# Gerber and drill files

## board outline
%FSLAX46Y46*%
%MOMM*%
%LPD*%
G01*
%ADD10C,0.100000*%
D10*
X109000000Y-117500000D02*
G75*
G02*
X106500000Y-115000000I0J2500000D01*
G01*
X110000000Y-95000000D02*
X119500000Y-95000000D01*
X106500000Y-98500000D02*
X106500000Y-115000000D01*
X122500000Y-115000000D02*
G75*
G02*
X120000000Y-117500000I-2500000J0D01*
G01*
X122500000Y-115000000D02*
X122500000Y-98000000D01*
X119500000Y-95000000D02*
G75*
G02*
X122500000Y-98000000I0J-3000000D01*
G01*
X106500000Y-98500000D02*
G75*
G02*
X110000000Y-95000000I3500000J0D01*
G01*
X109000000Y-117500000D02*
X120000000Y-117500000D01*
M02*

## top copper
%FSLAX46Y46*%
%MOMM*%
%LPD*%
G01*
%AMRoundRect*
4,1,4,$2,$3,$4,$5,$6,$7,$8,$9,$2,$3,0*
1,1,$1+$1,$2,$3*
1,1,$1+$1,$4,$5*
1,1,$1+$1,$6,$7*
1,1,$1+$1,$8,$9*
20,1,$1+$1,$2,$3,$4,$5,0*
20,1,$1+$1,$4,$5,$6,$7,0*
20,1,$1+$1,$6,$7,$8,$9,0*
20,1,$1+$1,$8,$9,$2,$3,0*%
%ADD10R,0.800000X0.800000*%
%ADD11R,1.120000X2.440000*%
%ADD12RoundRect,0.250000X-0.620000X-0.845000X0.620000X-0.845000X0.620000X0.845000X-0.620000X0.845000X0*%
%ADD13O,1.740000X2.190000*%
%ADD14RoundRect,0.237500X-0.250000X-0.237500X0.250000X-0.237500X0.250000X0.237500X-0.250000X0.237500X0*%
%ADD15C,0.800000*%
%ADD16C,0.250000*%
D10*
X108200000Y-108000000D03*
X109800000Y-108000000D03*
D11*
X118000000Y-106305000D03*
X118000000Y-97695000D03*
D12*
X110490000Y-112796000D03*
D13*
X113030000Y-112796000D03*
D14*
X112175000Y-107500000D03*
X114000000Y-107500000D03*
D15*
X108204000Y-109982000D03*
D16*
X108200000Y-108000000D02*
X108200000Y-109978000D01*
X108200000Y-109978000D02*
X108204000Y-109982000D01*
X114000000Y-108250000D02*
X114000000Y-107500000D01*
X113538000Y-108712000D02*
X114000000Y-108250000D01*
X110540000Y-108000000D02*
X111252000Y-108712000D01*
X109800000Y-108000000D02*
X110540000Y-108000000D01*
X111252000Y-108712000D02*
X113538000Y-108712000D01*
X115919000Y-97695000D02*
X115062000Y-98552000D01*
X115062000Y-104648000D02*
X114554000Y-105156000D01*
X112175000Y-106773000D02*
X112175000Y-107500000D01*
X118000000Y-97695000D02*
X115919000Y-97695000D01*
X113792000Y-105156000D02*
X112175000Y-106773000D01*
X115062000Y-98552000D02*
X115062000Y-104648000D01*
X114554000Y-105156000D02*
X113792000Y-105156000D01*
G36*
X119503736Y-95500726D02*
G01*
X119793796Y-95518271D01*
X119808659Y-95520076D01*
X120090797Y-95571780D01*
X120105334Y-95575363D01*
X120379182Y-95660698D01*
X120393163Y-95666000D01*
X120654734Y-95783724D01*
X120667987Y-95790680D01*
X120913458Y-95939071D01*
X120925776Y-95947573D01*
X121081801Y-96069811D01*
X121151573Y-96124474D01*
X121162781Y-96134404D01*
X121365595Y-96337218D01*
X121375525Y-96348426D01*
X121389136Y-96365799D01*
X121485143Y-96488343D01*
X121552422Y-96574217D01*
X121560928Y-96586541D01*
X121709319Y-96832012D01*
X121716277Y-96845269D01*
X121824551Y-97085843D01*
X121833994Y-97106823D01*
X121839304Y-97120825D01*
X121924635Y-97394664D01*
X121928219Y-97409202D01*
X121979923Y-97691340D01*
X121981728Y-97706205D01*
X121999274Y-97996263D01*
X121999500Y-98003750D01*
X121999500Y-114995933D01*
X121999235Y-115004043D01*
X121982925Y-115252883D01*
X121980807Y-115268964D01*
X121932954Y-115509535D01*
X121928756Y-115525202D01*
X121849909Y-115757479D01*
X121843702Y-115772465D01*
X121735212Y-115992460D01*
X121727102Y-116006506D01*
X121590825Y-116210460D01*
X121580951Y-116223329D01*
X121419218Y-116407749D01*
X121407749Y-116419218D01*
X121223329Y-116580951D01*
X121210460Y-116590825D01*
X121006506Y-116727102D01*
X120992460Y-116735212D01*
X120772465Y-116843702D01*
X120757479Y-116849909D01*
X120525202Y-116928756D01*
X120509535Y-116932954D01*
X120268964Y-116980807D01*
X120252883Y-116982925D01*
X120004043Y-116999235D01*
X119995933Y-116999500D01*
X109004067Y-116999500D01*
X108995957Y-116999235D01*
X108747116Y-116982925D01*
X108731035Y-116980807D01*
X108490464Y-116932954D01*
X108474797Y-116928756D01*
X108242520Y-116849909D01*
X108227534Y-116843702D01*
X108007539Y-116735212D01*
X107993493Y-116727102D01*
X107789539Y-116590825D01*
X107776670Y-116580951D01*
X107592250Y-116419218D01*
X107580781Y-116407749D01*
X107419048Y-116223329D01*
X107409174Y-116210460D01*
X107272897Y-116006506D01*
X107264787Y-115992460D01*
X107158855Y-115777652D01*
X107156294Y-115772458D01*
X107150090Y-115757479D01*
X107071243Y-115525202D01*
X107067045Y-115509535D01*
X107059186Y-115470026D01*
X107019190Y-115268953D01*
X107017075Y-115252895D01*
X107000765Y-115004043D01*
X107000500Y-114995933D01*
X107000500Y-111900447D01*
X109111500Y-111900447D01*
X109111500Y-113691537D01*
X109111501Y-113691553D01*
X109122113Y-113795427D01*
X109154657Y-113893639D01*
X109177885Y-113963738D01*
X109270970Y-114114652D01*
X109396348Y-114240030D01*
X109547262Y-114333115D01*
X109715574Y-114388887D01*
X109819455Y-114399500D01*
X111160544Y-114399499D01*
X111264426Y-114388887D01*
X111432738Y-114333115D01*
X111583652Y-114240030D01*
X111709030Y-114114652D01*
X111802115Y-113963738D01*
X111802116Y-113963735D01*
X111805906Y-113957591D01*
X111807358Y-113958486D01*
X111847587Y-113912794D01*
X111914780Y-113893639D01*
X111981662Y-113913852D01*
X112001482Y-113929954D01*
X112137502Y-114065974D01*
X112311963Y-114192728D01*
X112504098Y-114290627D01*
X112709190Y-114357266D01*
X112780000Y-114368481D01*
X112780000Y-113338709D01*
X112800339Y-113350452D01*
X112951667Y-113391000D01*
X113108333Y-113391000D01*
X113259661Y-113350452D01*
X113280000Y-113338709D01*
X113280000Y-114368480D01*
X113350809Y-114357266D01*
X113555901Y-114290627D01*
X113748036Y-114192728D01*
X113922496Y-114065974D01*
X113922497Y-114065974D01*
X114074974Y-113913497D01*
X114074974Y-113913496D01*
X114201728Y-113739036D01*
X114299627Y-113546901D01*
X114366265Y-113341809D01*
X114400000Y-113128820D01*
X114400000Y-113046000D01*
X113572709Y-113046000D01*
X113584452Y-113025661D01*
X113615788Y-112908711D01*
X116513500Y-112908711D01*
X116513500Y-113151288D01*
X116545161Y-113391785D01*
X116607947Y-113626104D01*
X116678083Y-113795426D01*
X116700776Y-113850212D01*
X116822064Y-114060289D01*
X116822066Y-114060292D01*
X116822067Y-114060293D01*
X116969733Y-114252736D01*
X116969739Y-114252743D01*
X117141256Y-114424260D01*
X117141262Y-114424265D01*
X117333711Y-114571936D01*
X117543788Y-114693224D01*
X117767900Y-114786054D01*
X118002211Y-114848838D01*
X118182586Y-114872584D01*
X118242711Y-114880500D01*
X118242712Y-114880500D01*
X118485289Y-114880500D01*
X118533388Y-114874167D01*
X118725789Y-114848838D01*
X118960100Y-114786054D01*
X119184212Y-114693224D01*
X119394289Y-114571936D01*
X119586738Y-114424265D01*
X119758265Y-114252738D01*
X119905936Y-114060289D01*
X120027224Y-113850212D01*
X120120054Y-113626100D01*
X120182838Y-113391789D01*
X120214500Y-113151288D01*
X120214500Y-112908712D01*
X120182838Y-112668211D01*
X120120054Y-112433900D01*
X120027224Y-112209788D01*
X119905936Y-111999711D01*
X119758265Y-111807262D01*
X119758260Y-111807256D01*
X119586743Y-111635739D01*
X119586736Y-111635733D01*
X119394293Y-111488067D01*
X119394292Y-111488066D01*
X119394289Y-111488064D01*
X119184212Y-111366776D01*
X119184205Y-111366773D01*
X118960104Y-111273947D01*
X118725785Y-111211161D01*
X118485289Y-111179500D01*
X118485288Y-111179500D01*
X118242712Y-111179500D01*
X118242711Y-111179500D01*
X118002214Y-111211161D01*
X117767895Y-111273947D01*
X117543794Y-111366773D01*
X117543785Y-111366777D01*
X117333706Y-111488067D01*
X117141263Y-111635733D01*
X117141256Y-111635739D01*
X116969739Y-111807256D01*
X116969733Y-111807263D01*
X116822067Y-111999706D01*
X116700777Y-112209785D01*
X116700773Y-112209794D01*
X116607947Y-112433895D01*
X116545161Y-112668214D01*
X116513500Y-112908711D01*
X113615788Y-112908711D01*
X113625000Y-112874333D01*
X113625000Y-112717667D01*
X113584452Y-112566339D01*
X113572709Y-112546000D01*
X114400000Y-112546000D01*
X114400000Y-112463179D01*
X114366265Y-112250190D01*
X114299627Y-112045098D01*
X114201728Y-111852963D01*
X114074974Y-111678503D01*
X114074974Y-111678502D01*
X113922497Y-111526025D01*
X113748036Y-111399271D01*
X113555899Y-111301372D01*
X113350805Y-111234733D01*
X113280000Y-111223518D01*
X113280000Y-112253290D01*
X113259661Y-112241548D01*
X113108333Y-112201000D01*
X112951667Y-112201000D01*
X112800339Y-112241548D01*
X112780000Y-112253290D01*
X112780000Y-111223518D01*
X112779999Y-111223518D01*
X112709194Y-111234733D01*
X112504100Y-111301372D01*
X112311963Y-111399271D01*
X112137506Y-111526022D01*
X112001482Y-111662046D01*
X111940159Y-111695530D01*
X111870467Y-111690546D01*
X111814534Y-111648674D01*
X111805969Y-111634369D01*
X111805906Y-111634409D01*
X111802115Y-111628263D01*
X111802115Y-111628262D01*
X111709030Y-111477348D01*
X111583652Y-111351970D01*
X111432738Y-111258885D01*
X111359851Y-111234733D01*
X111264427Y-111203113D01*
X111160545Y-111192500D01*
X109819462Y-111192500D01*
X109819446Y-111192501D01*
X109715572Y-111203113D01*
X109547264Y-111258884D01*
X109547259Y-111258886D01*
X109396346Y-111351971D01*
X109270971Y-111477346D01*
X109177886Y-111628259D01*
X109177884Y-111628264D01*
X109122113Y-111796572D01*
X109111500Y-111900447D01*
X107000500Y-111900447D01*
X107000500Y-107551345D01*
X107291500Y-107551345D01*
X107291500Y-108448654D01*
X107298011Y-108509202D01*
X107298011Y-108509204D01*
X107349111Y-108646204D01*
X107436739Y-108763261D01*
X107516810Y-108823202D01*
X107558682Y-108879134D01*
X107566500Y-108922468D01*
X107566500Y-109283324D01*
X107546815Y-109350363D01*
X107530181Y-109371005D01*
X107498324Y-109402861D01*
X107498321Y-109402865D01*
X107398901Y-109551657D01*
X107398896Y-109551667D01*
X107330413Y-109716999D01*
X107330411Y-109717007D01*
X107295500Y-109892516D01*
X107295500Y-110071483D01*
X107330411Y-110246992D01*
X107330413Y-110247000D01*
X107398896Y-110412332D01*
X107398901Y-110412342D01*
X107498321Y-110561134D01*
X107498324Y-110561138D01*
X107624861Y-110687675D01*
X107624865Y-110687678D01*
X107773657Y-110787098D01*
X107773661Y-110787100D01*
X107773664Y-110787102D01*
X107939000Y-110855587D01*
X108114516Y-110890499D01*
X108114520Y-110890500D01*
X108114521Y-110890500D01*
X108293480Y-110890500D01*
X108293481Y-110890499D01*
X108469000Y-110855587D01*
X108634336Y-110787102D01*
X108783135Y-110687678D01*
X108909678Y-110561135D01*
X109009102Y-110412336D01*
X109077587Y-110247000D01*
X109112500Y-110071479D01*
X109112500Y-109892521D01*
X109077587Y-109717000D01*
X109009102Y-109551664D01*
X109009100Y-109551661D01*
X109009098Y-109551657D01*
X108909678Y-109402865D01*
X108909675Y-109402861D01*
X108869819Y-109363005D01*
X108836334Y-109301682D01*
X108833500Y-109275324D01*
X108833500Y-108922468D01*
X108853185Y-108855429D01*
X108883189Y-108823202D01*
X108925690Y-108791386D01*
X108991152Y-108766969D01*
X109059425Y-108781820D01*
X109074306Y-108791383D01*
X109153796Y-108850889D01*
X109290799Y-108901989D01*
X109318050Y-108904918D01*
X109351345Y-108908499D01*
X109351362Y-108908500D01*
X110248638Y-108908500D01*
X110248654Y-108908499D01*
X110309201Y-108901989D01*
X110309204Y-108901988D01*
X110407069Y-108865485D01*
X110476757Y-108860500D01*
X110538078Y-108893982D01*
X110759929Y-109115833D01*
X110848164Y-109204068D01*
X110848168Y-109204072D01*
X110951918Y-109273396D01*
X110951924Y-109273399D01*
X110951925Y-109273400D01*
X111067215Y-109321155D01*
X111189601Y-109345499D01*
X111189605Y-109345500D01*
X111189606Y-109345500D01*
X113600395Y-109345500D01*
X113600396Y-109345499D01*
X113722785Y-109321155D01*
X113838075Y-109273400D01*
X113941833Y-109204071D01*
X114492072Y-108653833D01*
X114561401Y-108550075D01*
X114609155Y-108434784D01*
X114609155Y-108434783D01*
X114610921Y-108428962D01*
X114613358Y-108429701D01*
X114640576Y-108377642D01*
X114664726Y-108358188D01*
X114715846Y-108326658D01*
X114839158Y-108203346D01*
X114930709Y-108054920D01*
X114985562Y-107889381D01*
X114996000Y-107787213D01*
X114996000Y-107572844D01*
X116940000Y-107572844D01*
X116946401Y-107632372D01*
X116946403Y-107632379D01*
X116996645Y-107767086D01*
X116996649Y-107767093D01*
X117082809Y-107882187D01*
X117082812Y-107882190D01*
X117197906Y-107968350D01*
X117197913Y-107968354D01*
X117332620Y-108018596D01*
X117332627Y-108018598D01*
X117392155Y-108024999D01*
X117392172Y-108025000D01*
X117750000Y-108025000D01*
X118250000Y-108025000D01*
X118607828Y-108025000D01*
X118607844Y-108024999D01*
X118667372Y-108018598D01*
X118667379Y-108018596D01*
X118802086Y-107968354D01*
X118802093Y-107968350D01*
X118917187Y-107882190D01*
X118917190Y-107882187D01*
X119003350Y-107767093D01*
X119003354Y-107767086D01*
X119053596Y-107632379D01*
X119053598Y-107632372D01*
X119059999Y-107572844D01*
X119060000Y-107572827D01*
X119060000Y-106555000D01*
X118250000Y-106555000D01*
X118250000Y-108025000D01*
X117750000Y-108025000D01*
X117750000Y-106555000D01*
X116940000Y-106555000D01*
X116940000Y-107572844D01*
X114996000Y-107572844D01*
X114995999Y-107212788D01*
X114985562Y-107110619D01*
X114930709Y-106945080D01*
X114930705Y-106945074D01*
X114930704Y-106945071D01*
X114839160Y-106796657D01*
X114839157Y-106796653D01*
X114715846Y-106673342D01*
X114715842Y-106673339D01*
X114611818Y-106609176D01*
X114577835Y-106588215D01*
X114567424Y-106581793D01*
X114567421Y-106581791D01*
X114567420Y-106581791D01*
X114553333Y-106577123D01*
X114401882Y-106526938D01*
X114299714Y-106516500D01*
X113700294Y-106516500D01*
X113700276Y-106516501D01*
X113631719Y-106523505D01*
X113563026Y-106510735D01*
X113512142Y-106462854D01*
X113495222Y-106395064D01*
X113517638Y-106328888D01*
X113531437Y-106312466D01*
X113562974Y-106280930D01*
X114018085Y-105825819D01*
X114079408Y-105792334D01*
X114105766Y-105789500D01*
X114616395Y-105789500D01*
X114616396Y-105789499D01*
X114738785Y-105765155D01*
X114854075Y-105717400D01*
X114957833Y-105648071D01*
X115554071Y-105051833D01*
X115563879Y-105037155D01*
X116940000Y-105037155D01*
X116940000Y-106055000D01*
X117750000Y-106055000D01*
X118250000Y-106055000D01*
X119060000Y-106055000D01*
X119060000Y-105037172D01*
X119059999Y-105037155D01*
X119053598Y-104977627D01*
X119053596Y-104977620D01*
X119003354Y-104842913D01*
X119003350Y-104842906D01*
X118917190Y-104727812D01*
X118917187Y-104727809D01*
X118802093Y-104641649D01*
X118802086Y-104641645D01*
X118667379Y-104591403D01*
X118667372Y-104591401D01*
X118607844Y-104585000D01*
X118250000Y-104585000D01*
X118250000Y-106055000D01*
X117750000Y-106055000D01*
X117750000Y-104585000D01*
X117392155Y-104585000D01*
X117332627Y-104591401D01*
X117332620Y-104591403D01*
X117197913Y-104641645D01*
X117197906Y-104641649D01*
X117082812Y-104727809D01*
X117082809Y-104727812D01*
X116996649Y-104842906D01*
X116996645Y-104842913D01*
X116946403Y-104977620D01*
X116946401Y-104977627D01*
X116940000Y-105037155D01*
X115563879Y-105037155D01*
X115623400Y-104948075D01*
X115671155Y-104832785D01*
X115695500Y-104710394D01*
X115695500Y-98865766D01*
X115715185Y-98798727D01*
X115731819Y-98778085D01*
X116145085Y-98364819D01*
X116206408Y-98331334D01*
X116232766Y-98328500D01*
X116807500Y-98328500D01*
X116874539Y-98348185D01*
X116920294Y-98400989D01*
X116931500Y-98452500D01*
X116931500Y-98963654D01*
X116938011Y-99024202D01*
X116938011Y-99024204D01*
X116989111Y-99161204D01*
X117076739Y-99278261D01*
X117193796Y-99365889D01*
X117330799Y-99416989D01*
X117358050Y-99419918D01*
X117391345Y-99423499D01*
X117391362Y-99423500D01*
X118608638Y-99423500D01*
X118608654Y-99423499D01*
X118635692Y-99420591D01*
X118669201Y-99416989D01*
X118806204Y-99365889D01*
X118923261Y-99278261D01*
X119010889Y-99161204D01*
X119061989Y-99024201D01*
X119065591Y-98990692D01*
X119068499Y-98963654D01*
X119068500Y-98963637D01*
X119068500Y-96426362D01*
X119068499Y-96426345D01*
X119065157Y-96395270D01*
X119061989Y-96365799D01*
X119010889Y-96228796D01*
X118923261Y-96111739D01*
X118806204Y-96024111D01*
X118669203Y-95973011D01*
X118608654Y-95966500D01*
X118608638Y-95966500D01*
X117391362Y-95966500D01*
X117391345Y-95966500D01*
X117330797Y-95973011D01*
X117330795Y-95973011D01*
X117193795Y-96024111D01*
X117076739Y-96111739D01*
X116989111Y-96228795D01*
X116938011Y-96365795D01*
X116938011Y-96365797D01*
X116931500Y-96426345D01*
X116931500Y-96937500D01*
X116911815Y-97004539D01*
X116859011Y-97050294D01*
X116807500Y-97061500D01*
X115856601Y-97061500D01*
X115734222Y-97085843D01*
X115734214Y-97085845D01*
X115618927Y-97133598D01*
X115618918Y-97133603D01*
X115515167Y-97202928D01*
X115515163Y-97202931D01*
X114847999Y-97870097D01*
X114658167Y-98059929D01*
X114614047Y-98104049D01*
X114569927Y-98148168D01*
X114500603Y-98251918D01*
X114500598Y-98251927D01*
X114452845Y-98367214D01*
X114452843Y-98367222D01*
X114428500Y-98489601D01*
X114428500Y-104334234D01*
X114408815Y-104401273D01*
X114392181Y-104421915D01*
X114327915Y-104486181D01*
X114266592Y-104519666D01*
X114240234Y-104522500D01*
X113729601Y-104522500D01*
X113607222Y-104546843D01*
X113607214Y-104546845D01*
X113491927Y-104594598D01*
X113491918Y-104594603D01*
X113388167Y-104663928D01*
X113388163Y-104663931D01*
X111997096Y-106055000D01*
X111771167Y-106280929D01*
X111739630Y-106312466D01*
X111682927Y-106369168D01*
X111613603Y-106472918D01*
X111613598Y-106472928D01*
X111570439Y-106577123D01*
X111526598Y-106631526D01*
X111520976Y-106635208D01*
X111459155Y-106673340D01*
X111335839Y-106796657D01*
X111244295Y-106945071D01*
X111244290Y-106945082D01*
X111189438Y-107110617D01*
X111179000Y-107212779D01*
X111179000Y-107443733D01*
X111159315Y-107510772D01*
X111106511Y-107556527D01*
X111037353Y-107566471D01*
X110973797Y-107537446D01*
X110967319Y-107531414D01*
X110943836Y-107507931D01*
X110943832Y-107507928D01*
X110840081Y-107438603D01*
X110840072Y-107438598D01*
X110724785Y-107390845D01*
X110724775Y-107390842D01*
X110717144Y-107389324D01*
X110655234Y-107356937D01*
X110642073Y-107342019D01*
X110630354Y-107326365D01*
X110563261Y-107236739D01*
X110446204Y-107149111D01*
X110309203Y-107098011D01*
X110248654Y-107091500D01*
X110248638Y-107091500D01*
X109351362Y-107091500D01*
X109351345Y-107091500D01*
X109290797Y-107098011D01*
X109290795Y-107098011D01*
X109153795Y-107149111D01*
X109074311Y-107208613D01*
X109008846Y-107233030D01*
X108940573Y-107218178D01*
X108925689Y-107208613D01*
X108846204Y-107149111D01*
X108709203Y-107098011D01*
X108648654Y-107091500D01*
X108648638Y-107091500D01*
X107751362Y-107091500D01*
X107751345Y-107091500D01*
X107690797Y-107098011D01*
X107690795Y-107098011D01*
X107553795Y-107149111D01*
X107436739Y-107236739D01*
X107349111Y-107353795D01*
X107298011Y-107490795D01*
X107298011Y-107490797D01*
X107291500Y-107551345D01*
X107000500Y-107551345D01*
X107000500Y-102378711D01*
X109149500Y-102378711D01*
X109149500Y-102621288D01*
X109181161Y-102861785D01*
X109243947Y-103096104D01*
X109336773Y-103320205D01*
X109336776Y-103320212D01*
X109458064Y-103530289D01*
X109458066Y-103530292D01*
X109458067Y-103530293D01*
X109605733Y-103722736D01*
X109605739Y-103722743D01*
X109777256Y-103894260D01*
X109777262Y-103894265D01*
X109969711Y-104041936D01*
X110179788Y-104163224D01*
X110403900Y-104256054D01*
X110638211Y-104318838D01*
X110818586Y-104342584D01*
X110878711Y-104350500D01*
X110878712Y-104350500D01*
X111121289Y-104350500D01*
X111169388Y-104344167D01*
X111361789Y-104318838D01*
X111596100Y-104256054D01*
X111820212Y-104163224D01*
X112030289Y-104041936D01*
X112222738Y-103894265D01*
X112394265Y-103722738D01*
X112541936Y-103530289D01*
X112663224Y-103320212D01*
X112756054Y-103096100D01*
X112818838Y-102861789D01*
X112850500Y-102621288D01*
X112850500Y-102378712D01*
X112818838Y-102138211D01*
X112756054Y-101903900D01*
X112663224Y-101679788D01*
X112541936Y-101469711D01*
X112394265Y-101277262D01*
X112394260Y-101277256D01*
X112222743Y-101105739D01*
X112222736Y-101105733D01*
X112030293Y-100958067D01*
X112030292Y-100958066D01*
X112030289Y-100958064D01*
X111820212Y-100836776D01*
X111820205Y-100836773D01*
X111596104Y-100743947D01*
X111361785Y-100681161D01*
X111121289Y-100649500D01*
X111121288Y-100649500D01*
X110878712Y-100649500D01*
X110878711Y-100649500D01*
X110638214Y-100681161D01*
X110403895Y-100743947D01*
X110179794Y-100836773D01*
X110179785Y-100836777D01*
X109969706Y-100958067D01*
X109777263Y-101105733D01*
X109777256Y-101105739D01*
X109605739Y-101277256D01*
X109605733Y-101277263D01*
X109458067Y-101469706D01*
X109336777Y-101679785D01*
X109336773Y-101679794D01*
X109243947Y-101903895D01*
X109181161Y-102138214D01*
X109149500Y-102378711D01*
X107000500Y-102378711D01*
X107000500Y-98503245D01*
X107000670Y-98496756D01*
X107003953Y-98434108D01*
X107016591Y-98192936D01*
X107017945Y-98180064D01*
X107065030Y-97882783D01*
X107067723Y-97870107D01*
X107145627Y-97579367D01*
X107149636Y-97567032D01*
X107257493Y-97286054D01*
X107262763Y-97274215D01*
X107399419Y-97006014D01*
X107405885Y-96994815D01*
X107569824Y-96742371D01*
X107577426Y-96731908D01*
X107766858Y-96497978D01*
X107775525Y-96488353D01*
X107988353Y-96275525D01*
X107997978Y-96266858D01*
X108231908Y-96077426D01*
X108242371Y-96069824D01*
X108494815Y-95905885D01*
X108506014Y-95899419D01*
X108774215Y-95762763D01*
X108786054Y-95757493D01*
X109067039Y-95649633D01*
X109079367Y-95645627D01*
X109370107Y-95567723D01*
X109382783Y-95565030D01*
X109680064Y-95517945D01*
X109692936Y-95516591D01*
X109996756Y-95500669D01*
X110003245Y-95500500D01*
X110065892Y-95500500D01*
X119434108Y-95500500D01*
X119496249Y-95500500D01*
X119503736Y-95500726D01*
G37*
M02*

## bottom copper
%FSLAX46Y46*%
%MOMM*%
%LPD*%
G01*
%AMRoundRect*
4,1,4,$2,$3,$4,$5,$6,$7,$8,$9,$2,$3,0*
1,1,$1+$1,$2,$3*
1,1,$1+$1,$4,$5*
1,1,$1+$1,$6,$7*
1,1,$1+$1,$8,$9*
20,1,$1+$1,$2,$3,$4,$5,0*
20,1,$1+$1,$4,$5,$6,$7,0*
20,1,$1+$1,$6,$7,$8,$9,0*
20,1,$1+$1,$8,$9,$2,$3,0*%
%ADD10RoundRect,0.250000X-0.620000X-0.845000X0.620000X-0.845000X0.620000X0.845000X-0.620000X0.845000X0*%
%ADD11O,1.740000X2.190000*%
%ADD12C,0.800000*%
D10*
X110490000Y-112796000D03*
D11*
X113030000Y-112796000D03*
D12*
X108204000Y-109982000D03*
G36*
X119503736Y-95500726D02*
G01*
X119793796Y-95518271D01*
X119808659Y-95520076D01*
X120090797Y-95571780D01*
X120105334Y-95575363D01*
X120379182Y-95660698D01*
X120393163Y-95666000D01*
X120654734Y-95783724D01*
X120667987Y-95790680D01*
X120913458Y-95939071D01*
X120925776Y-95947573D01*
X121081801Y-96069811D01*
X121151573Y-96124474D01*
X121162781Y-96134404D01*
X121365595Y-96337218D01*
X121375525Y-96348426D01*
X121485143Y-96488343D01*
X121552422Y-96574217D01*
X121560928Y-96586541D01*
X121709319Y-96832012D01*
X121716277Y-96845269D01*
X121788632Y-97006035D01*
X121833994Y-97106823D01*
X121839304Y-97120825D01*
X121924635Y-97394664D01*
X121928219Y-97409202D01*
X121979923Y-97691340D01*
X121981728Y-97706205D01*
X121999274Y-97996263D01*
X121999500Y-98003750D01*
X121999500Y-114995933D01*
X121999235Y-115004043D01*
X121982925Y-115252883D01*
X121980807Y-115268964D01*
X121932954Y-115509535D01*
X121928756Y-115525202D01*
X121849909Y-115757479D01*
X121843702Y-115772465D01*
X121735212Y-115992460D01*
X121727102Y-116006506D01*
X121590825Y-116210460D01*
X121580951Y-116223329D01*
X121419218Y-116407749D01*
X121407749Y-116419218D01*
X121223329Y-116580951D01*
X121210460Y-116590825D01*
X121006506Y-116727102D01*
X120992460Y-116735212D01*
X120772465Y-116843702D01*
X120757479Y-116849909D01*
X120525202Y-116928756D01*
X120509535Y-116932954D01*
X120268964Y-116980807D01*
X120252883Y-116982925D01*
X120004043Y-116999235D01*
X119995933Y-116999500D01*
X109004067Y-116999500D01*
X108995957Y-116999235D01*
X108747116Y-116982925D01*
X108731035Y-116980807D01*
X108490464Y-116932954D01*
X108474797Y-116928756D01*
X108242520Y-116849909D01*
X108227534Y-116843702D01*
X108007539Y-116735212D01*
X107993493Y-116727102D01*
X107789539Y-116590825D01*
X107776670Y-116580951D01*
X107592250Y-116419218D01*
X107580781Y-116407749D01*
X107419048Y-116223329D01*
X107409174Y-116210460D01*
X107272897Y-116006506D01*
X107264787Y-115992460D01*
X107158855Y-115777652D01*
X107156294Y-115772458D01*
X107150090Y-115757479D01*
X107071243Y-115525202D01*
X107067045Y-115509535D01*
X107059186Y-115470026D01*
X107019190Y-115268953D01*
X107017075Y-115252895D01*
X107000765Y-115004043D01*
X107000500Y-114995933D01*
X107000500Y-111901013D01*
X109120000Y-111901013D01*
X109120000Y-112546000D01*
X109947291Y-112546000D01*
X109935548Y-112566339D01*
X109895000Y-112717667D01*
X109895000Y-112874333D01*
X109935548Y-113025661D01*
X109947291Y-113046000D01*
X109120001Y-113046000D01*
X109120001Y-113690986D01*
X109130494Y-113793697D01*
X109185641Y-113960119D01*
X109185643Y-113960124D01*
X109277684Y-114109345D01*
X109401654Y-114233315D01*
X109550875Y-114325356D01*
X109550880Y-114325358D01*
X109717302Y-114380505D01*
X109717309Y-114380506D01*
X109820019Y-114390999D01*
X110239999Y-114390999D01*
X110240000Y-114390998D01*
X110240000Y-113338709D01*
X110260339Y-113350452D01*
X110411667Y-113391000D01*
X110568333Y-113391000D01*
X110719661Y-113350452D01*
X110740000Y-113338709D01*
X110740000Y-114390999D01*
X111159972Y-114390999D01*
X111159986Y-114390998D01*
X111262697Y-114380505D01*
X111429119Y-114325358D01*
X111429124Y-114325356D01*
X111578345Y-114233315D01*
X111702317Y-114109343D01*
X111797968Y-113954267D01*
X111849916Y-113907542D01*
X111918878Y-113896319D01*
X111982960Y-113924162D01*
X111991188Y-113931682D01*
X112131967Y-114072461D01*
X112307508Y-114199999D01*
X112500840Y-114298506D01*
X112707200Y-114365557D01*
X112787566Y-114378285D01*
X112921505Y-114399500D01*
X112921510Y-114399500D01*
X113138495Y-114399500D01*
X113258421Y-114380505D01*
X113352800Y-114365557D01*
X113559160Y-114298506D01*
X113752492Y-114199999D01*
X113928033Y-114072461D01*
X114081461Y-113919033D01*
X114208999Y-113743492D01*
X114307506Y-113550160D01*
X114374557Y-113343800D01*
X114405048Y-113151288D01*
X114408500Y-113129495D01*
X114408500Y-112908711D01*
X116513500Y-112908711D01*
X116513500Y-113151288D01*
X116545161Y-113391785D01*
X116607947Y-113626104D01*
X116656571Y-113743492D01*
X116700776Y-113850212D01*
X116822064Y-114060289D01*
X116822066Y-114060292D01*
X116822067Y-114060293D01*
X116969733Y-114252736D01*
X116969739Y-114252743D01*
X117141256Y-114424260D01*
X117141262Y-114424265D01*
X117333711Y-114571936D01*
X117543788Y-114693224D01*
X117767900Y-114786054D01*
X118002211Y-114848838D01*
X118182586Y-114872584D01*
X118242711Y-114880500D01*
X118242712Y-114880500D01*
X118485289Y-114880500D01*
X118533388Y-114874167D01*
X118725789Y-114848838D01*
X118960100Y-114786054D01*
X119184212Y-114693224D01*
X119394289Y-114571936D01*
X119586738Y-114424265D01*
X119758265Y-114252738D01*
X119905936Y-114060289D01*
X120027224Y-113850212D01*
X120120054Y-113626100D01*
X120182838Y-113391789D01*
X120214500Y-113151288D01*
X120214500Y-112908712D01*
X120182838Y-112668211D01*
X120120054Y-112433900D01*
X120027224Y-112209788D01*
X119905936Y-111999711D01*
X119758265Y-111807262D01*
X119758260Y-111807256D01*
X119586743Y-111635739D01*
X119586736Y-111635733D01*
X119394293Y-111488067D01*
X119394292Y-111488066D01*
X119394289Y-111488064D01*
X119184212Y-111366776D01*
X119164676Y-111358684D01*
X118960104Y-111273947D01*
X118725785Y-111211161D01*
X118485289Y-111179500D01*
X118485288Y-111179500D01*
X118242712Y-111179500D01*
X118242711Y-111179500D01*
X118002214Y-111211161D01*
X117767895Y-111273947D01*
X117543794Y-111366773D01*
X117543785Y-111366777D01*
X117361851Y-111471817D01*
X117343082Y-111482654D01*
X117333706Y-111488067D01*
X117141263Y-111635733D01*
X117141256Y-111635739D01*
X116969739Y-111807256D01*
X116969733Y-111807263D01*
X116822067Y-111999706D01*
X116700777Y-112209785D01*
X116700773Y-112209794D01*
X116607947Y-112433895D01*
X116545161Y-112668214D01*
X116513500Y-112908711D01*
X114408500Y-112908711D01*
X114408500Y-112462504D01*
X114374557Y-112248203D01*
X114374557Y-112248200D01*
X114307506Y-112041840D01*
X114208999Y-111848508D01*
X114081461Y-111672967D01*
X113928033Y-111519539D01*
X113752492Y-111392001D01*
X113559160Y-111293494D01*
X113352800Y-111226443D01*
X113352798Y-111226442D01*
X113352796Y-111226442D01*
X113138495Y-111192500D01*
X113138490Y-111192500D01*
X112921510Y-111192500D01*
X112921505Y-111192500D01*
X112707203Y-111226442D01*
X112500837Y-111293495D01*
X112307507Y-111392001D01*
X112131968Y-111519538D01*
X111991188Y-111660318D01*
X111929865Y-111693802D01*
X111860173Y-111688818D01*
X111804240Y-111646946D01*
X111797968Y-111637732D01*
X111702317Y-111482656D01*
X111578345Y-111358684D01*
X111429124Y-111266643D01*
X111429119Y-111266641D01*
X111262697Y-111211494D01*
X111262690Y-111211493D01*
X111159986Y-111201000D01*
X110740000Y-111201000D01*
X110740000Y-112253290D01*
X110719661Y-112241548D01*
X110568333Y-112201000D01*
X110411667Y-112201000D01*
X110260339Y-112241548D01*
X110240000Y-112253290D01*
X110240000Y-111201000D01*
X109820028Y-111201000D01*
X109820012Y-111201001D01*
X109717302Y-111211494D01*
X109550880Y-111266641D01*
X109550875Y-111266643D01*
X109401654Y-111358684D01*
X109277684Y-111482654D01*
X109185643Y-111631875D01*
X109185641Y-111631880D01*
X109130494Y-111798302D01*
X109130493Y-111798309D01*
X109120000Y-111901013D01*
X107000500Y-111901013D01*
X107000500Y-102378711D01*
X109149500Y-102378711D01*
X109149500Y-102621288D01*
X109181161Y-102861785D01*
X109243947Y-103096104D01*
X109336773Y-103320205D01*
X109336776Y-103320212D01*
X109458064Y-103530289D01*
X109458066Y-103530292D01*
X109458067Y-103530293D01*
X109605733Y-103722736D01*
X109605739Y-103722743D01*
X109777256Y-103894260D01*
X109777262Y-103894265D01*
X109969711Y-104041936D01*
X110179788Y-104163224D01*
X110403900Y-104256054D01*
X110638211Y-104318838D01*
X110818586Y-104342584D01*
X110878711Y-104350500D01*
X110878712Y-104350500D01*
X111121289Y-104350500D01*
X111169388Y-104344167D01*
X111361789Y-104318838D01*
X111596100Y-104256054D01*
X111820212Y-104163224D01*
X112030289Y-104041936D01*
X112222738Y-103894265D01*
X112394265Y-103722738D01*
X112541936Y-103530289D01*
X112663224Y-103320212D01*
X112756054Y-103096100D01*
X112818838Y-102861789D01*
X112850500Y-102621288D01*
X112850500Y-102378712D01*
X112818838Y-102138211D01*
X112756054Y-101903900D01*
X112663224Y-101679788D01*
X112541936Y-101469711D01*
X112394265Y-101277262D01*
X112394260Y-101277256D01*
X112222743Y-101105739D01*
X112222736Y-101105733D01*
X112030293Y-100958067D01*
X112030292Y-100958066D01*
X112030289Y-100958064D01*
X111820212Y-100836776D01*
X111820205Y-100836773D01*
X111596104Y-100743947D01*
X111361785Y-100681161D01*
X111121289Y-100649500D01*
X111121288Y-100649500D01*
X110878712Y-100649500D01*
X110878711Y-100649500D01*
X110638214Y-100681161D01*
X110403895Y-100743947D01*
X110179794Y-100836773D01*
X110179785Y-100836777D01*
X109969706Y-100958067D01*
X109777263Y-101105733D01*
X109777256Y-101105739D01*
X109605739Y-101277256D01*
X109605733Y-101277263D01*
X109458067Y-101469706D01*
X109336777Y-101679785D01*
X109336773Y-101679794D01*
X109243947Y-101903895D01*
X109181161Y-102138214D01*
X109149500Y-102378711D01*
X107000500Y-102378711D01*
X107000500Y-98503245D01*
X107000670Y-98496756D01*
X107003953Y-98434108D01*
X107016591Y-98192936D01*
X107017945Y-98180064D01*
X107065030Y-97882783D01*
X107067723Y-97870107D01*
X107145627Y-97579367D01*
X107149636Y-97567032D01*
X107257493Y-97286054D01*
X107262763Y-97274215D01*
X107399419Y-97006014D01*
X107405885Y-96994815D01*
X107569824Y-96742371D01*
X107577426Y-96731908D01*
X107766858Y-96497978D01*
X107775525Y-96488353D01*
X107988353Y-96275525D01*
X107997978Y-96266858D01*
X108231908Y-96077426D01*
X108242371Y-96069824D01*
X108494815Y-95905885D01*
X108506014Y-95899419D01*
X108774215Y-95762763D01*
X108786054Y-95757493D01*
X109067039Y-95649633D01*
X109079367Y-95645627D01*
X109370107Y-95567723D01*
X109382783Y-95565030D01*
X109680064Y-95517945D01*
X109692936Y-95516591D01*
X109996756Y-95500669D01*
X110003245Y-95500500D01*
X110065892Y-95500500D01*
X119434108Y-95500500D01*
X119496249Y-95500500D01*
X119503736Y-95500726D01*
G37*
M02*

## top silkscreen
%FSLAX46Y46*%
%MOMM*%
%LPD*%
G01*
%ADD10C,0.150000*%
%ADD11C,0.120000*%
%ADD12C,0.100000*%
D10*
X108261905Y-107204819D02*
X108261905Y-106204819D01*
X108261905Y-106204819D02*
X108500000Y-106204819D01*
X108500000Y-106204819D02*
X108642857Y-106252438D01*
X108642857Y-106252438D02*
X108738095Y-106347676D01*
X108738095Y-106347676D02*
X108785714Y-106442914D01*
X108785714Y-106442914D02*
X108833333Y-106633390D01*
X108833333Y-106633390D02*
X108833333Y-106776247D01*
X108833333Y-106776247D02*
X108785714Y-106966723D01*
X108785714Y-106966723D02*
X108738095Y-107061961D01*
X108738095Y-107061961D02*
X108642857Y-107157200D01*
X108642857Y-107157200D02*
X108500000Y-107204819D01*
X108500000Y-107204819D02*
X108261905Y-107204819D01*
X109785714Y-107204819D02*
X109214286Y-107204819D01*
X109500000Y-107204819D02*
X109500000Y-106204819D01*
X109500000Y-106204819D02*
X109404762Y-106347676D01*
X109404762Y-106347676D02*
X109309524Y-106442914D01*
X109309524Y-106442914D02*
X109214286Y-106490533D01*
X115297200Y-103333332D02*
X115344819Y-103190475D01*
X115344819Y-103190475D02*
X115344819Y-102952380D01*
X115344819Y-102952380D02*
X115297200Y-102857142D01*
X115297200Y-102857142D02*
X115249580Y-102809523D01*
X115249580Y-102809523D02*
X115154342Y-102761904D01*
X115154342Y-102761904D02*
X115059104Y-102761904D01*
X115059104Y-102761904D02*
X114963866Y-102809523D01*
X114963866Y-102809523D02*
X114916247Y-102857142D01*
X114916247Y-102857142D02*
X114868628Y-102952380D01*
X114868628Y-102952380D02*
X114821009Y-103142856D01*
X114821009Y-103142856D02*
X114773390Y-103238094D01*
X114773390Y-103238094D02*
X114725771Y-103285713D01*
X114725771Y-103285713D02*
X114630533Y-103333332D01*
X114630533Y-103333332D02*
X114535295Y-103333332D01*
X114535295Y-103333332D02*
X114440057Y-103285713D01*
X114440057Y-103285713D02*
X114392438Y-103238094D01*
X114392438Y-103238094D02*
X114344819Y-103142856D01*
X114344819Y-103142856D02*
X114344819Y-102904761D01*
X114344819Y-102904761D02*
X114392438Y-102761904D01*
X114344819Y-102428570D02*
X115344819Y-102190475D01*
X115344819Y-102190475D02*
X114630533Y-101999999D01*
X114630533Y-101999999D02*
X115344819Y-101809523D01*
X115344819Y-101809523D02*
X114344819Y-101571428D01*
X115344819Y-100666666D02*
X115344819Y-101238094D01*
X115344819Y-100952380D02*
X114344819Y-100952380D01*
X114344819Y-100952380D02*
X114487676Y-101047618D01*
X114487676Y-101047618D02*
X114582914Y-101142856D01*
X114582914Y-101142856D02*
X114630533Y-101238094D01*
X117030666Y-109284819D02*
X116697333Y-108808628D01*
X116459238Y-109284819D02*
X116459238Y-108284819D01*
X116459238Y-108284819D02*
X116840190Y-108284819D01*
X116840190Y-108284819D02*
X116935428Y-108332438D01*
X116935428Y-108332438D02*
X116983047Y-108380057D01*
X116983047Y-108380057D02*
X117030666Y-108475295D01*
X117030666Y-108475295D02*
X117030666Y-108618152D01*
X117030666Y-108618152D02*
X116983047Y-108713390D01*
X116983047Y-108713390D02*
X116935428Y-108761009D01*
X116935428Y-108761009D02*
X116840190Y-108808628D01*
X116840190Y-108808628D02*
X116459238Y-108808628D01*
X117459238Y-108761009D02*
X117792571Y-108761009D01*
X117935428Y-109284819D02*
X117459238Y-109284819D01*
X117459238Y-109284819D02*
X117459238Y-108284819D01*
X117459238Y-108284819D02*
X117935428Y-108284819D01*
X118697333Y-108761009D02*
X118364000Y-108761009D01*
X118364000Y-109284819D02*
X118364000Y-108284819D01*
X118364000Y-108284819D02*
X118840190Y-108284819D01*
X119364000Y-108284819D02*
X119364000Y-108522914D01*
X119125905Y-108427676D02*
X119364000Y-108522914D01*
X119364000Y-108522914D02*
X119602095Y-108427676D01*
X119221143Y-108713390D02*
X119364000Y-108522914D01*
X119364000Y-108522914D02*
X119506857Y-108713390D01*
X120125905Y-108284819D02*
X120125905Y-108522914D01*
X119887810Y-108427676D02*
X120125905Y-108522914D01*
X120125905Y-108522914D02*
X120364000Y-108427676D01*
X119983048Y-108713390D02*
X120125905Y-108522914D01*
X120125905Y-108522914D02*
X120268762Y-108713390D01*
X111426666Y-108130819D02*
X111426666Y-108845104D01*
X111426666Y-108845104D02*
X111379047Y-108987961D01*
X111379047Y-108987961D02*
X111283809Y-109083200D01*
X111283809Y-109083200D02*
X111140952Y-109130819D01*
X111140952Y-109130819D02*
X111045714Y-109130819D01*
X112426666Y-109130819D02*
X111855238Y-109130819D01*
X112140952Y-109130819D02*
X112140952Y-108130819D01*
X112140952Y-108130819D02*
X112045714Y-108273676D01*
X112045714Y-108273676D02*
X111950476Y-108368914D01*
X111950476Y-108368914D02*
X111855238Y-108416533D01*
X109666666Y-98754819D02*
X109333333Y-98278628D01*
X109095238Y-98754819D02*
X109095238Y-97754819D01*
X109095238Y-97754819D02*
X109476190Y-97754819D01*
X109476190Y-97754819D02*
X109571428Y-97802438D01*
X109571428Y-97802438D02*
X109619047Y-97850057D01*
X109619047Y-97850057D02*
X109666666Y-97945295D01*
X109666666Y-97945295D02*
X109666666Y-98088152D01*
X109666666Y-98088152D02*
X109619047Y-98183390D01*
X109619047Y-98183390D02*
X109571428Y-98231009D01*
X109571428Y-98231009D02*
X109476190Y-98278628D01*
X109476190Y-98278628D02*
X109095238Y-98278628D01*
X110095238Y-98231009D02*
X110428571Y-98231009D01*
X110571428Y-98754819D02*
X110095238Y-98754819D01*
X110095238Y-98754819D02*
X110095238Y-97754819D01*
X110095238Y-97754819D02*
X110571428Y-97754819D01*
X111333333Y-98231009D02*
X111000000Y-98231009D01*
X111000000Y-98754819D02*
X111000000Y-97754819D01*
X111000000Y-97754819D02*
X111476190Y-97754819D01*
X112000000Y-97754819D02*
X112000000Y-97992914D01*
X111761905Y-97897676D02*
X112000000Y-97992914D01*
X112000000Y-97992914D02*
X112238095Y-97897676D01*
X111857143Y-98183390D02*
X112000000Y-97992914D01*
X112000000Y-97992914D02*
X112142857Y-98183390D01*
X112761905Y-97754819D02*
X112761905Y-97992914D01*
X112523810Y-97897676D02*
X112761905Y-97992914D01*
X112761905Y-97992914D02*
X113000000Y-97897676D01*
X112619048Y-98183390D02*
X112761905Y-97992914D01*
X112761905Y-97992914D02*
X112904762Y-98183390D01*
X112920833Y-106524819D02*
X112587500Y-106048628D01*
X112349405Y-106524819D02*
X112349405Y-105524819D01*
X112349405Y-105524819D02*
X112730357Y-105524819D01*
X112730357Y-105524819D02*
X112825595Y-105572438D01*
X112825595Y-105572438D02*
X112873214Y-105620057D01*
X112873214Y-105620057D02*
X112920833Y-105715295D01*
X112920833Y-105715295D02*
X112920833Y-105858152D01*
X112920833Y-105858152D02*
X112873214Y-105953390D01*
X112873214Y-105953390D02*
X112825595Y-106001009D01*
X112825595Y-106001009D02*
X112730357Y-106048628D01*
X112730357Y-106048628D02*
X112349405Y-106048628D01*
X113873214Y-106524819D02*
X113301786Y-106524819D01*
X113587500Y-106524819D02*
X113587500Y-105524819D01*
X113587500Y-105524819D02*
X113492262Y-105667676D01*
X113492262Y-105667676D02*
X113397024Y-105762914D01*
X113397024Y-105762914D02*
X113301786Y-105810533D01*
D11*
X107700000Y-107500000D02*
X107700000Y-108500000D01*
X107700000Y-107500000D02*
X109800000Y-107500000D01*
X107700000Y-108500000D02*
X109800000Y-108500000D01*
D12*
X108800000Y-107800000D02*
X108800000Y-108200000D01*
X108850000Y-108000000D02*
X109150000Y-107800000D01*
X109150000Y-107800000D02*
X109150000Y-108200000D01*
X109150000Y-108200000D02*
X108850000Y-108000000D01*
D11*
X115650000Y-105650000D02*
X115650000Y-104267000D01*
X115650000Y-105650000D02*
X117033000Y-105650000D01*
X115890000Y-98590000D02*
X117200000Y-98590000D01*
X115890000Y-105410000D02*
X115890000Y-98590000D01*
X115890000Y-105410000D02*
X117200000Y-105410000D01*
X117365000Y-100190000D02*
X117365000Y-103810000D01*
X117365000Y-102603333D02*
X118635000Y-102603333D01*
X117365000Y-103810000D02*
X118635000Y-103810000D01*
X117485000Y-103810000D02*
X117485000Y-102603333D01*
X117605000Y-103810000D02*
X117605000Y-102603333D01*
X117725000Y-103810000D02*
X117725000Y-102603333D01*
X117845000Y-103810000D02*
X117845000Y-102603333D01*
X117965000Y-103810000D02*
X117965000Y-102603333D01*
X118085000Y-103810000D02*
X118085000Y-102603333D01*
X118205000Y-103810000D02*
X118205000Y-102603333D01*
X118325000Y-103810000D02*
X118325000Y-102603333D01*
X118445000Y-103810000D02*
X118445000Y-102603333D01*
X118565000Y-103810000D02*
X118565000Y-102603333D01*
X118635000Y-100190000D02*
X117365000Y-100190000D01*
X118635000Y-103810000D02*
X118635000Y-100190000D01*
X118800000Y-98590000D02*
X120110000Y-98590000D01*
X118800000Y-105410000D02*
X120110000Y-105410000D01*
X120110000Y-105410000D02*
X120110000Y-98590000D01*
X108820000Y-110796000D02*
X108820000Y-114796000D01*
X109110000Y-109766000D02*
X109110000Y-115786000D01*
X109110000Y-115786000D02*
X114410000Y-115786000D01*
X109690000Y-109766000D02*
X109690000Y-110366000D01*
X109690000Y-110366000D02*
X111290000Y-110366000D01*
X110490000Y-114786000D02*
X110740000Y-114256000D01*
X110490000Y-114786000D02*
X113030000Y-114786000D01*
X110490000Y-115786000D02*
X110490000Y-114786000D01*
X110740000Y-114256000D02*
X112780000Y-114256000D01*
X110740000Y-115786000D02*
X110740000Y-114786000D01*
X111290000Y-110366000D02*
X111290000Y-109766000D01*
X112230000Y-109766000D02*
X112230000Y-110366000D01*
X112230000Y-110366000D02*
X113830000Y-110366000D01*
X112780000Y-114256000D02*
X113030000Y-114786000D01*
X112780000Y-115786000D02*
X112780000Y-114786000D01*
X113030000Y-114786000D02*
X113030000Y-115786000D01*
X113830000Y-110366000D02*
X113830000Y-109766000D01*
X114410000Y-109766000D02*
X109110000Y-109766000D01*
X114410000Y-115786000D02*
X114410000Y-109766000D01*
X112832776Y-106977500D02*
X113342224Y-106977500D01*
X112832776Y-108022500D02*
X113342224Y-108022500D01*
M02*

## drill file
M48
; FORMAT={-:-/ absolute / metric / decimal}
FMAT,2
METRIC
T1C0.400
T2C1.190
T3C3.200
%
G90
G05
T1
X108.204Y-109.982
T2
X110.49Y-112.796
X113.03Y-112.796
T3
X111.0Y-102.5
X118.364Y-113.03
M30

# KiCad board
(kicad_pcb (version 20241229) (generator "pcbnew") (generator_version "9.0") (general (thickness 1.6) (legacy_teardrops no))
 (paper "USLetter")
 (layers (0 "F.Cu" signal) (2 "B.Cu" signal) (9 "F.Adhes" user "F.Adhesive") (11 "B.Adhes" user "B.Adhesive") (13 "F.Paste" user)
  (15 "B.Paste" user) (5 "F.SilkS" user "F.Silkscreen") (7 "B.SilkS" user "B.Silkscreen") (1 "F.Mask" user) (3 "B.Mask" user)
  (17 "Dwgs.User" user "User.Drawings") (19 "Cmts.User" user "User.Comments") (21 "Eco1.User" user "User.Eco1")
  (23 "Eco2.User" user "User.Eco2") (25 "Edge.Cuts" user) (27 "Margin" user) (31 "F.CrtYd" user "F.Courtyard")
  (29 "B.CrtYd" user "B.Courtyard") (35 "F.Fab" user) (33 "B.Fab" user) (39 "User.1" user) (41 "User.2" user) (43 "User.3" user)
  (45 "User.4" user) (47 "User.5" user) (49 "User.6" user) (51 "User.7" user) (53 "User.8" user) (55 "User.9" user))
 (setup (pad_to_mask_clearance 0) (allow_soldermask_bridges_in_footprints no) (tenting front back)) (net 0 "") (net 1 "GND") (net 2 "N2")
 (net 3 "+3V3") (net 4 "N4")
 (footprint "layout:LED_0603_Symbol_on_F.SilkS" (layer "F.Cu") (at 109 108)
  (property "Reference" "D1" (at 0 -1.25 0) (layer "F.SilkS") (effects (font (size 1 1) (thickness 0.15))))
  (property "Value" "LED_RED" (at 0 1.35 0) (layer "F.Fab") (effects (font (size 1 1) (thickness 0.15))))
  (fp_line (start -1.3 -0.5) (end -1.3 0.5) (stroke (width 0.12) (type solid)) (layer "F.SilkS"))
  (fp_line (start -1.3 -0.5) (end 0.8 -0.5) (stroke (width 0.12) (type solid)) (layer "F.SilkS"))
  (fp_line (start -1.3 0.5) (end 0.8 0.5) (stroke (width 0.12) (type solid)) (layer "F.SilkS"))
  (fp_line (start -0.2 -0.2) (end -0.2 0.2) (stroke (width 0.1) (type solid)) (layer "F.SilkS"))
  (fp_line (start -0.15 0) (end 0.15 -0.2) (stroke (width 0.1) (type solid)) (layer "F.SilkS"))
  (fp_line (start 0.15 -0.2) (end 0.15 0.2) (stroke (width 0.1) (type solid)) (layer "F.SilkS"))
  (fp_line (start 0.15 0.2) (end -0.15 0) (stroke (width 0.1) (type solid)) (layer "F.SilkS"))
  (pad "1" smd rect (at -0.8 0 180) (size 0.8 0.8) (layers "F.Cu" "F.Mask" "F.Paste") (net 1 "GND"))
  (pad "2" smd rect (at 0.8 0 180) (size 0.8 0.8) (layers "F.Cu" "F.Mask" "F.Paste") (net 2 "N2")))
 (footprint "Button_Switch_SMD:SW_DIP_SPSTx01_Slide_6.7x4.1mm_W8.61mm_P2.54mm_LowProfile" (layer "F.Cu") (at 118 102 90)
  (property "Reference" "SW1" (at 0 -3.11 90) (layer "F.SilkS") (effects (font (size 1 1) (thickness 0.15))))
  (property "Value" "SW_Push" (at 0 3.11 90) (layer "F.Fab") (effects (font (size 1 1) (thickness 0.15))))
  (fp_line (start -3.65 -2.35) (end -2.267 -2.35) (stroke (width 0.12) (type solid)) (layer "F.SilkS"))
  (fp_line (start -3.65 -2.35) (end -3.65 -0.967) (stroke (width 0.12) (type solid)) (layer "F.SilkS"))
  (fp_line (start 3.41 -2.11) (end 3.41 -0.8) (stroke (width 0.12) (type solid)) (layer "F.SilkS"))
  (fp_line (start -3.41 -2.11) (end 3.41 -2.11) (stroke (width 0.12) (type solid)) (layer "F.SilkS"))
  (fp_line (start -3.41 -2.11) (end -3.41 -0.8) (stroke (width 0.12) (type solid)) (layer "F.SilkS"))
  (fp_line (start 1.81 -0.635) (end -1.81 -0.635) (stroke (width 0.12) (type solid)) (layer "F.SilkS"))
  (fp_line (start -0.603333 -0.635) (end -0.603333 0.635) (stroke (width 0.12) (type solid)) (layer "F.SilkS"))
  (fp_line (start -1.81 -0.635) (end -1.81 0.635) (stroke (width 0.12) (type solid)) (layer "F.SilkS"))
  (fp_line (start -1.81 -0.515) (end -0.603333 -0.515) (stroke (width 0.12) (type solid)) (layer "F.SilkS"))
  (fp_line (start -1.81 -0.395) (end -0.603333 -0.395) (stroke (width 0.12) (type solid)) (layer "F.SilkS"))
  (fp_line (start -1.81 -0.275) (end -0.603333 -0.275) (stroke (width 0.12) (type solid)) (layer "F.SilkS"))
  (fp_line (start -1.81 -0.155) (end -0.603333 -0.155) (stroke (width 0.12) (type solid)) (layer "F.SilkS"))
  (fp_line (start -1.81 -0.035) (end -0.603333 -0.035) (stroke (width 0.12) (type solid)) (layer "F.SilkS"))
  (fp_line (start -1.81 0.085) (end -0.603333 0.085) (stroke (width 0.12) (type solid)) (layer "F.SilkS"))
  (fp_line (start -1.81 0.205) (end -0.603333 0.205) (stroke (width 0.12) (type solid)) (layer "F.SilkS"))
  (fp_line (start -1.81 0.325) (end -0.603333 0.325) (stroke (width 0.12) (type solid)) (layer "F.SilkS"))
  (fp_line (start -1.81 0.445) (end -0.603333 0.445) (stroke (width 0.12) (type solid)) (layer "F.SilkS"))
  (fp_line (start -1.81 0.565) (end -0.603333 0.565) (stroke (width 0.12) (type solid)) (layer "F.SilkS"))
  (fp_line (start 1.81 0.635) (end 1.81 -0.635) (stroke (width 0.12) (type solid)) (layer "F.SilkS"))
  (fp_line (start -1.81 0.635) (end 1.81 0.635) (stroke (width 0.12) (type solid)) (layer "F.SilkS"))
  (fp_line (start 3.41 0.8) (end 3.41 2.11) (stroke (width 0.12) (type solid)) (layer "F.SilkS"))
  (fp_line (start -3.41 0.8) (end -3.41 2.11) (stroke (width 0.12) (type solid)) (layer "F.SilkS"))
  (fp_line (start -3.41 2.11) (end 3.41 2.11) (stroke (width 0.12) (type solid)) (layer "F.SilkS"))
  (pad "1" smd rect (at -4.305 0 90) (size 2.44 1.12) (layers "F.Cu" "F.Mask" "F.Paste") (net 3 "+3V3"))
  (pad "2" smd rect (at 4.305 0 90) (size 2.44 1.12) (layers "F.Cu" "F.Mask" "F.Paste") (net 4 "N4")))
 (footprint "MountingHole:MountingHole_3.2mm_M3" (layer "F.Cu") (at 118.364 113.03)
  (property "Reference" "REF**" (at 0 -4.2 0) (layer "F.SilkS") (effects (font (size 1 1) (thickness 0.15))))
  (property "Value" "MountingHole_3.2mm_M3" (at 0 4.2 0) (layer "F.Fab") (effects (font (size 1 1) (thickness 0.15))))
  (pad "" np_thru_hole circle (at 0 0) (size 3.2 3.2) (drill 3.2) (layers "*.Cu" "*.Mask")))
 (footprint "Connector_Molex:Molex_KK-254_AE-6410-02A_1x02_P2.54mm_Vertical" (layer "F.Cu") (at 110.49 112.796)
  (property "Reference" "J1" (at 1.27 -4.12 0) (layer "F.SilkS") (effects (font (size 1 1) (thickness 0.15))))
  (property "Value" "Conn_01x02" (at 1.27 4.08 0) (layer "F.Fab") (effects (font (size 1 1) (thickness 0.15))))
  (fp_line (start -1.67 -2) (end -1.67 2) (stroke (width 0.12) (type solid)) (layer "F.SilkS"))
  (fp_line (start -1.38 -3.03) (end -1.38 2.99) (stroke (width 0.12) (type solid)) (layer "F.SilkS"))
  (fp_line (start -1.38 2.99) (end 3.92 2.99) (stroke (width 0.12) (type solid)) (layer "F.SilkS"))
  (fp_line (start -0.8 -3.03) (end -0.8 -2.43) (stroke (width 0.12) (type solid)) (layer "F.SilkS"))
  (fp_line (start -0.8 -2.43) (end 0.8 -2.43) (stroke (width 0.12) (type solid)) (layer "F.SilkS"))
  (fp_line (start 0 1.99) (end 0.25 1.46) (stroke (width 0.12) (type solid)) (layer "F.SilkS"))
  (fp_line (start 0 1.99) (end 2.54 1.99) (stroke (width 0.12) (type solid)) (layer "F.SilkS"))
  (fp_line (start 0 2.99) (end 0 1.99) (stroke (width 0.12) (type solid)) (layer "F.SilkS"))
  (fp_line (start 0.25 1.46) (end 2.29 1.46) (stroke (width 0.12) (type solid)) (layer "F.SilkS"))
  (fp_line (start 0.25 2.99) (end 0.25 1.99) (stroke (width 0.12) (type solid)) (layer "F.SilkS"))
  (fp_line (start 0.8 -2.43) (end 0.8 -3.03) (stroke (width 0.12) (type solid)) (layer "F.SilkS"))
  (fp_line (start 1.74 -3.03) (end 1.74 -2.43) (stroke (width 0.12) (type solid)) (layer "F.SilkS"))
  (fp_line (start 1.74 -2.43) (end 3.34 -2.43) (stroke (width 0.12) (type solid)) (layer "F.SilkS"))
  (fp_line (start 2.29 1.46) (end 2.54 1.99) (stroke (width 0.12) (type solid)) (layer "F.SilkS"))
  (fp_line (start 2.29 2.99) (end 2.29 1.99) (stroke (width 0.12) (type solid)) (layer "F.SilkS"))
  (fp_line (start 2.54 1.99) (end 2.54 2.99) (stroke (width 0.12) (type solid)) (layer "F.SilkS"))
  (fp_line (start 3.34 -2.43) (end 3.34 -3.03) (stroke (width 0.12) (type solid)) (layer "F.SilkS"))
  (fp_line (start 3.92 -3.03) (end -1.38 -3.03) (stroke (width 0.12) (type solid)) (layer "F.SilkS"))
  (fp_line (start 3.92 2.99) (end 3.92 -3.03) (stroke (width 0.12) (type solid)) (layer "F.SilkS"))
  (pad "1" thru_hole roundrect (at 0 0) (size 1.74 2.19) (drill 1.19) (layers "*.Cu" "*.Mask") (remove_unused_layers no)
   (roundrect_rratio 0.143678) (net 1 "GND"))
  (pad "2" thru_hole oval (at 2.54 0) (size 1.74 2.19) (drill 1.19) (layers "*.Cu" "*.Mask") (remove_unused_layers no) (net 3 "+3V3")))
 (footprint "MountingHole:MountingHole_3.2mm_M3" (layer "F.Cu") (at 111 102.5)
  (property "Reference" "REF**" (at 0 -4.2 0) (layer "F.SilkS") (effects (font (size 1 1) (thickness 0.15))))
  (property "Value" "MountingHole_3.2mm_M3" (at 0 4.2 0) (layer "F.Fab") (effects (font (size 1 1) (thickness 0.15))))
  (pad "" np_thru_hole circle (at 0 0) (size 3.2 3.2) (drill 3.2) (layers "*.Cu" "*.Mask")))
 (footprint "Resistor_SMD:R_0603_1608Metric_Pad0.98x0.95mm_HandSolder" (layer "F.Cu") (at 113.0875 107.5)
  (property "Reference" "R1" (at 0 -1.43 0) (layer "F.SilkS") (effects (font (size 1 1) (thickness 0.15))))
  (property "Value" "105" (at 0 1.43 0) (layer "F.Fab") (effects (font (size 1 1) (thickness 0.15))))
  (fp_line (start -0.254724 -0.5225) (end 0.254724 -0.5225) (stroke (width 0.12) (type solid)) (layer "F.SilkS"))
  (fp_line (start -0.254724 0.5225) (end 0.254724 0.5225) (stroke (width 0.12) (type solid)) (layer "F.SilkS"))
  (pad "1" smd roundrect (at -0.9125 0) (size 0.975 0.95) (layers "F.Cu" "F.Mask" "F.Paste") (roundrect_rratio 0.25) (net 4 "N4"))
  (pad "2" smd roundrect (at 0.9125 0) (size 0.975 0.95) (layers "F.Cu" "F.Mask" "F.Paste") (roundrect_rratio 0.25) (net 2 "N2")))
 (gr_arc (start 109 117.5) (mid 107.232233 116.767767) (end 106.5 115) (stroke (width 0.1) (type default)) (layer "Edge.Cuts"))
 (gr_line (start 110 95) (end 119.5 95) (stroke (width 0.1) (type default)) (layer "Edge.Cuts"))
 (gr_line (start 106.5 98.5) (end 106.5 115) (stroke (width 0.1) (type default)) (layer "Edge.Cuts"))
 (gr_arc (start 122.5 115) (mid 121.767767 116.767767) (end 120 117.5) (stroke (width 0.1) (type default)) (layer "Edge.Cuts"))
 (gr_line (start 122.5 115) (end 122.5 98) (stroke (width 0.1) (type default)) (layer "Edge.Cuts"))
 (gr_arc (start 119.5 95) (mid 121.62132 95.87868) (end 122.5 98) (stroke (width 0.1) (type default)) (layer "Edge.Cuts"))
 (gr_arc (start 106.5 98.5) (mid 107.525126 96.025126) (end 110 95) (stroke (width 0.1) (type default)) (layer "Edge.Cuts"))
 (gr_line (start 109 117.5) (end 120 117.5) (stroke (width 0.1) (type default)) (layer "Edge.Cuts"))
 (segment (start 108.2 108) (end 108.2 109.978) (width 0.25) (layer "F.Cu") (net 1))
 (segment (start 108.2 109.978) (end 108.204 109.982) (width 0.25) (layer "F.Cu") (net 1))
 (via (at 108.204 109.982) (size 0.8) (drill 0.4) (layers "F.Cu" "B.Cu") (free yes) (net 1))
 (segment (start 114 108.25) (end 114 107.5) (width 0.25) (layer "F.Cu") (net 2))
 (segment (start 113.538 108.712) (end 114 108.25) (width 0.25) (layer "F.Cu") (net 2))
 (segment (start 110.54 108) (end 111.252 108.712) (width 0.25) (layer "F.Cu") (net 2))
 (segment (start 109.8 108) (end 110.54 108) (width 0.25) (layer "F.Cu") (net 2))
 (segment (start 111.252 108.712) (end 113.538 108.712) (width 0.25) (layer "F.Cu") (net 2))
 (segment (start 115.919 97.695) (end 115.062 98.552) (width 0.25) (layer "F.Cu") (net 4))
 (segment (start 115.062 104.648) (end 114.554 105.156) (width 0.25) (layer "F.Cu") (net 4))
 (segment (start 112.175 106.773) (end 112.175 107.5) (width 0.25) (layer "F.Cu") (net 4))
 (segment (start 118 97.695) (end 115.919 97.695) (width 0.25) (layer "F.Cu") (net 4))
 (segment (start 113.792 105.156) (end 112.175 106.773) (width 0.25) (layer "F.Cu") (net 4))
 (segment (start 115.062 98.552) (end 115.062 104.648) (width 0.25) (layer "F.Cu") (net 4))
 (segment (start 114.554 105.156) (end 113.792 105.156) (width 0.25) (layer "F.Cu") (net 4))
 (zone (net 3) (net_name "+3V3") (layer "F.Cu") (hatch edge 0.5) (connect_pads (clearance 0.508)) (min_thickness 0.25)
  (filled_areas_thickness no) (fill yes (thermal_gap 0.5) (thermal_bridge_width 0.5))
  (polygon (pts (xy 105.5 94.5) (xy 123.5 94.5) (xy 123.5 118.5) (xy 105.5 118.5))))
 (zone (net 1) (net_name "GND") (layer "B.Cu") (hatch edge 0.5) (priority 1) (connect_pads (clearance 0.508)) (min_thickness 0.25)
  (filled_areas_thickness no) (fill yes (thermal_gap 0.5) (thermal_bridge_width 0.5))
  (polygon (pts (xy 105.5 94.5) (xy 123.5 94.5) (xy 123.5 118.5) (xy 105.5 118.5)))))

